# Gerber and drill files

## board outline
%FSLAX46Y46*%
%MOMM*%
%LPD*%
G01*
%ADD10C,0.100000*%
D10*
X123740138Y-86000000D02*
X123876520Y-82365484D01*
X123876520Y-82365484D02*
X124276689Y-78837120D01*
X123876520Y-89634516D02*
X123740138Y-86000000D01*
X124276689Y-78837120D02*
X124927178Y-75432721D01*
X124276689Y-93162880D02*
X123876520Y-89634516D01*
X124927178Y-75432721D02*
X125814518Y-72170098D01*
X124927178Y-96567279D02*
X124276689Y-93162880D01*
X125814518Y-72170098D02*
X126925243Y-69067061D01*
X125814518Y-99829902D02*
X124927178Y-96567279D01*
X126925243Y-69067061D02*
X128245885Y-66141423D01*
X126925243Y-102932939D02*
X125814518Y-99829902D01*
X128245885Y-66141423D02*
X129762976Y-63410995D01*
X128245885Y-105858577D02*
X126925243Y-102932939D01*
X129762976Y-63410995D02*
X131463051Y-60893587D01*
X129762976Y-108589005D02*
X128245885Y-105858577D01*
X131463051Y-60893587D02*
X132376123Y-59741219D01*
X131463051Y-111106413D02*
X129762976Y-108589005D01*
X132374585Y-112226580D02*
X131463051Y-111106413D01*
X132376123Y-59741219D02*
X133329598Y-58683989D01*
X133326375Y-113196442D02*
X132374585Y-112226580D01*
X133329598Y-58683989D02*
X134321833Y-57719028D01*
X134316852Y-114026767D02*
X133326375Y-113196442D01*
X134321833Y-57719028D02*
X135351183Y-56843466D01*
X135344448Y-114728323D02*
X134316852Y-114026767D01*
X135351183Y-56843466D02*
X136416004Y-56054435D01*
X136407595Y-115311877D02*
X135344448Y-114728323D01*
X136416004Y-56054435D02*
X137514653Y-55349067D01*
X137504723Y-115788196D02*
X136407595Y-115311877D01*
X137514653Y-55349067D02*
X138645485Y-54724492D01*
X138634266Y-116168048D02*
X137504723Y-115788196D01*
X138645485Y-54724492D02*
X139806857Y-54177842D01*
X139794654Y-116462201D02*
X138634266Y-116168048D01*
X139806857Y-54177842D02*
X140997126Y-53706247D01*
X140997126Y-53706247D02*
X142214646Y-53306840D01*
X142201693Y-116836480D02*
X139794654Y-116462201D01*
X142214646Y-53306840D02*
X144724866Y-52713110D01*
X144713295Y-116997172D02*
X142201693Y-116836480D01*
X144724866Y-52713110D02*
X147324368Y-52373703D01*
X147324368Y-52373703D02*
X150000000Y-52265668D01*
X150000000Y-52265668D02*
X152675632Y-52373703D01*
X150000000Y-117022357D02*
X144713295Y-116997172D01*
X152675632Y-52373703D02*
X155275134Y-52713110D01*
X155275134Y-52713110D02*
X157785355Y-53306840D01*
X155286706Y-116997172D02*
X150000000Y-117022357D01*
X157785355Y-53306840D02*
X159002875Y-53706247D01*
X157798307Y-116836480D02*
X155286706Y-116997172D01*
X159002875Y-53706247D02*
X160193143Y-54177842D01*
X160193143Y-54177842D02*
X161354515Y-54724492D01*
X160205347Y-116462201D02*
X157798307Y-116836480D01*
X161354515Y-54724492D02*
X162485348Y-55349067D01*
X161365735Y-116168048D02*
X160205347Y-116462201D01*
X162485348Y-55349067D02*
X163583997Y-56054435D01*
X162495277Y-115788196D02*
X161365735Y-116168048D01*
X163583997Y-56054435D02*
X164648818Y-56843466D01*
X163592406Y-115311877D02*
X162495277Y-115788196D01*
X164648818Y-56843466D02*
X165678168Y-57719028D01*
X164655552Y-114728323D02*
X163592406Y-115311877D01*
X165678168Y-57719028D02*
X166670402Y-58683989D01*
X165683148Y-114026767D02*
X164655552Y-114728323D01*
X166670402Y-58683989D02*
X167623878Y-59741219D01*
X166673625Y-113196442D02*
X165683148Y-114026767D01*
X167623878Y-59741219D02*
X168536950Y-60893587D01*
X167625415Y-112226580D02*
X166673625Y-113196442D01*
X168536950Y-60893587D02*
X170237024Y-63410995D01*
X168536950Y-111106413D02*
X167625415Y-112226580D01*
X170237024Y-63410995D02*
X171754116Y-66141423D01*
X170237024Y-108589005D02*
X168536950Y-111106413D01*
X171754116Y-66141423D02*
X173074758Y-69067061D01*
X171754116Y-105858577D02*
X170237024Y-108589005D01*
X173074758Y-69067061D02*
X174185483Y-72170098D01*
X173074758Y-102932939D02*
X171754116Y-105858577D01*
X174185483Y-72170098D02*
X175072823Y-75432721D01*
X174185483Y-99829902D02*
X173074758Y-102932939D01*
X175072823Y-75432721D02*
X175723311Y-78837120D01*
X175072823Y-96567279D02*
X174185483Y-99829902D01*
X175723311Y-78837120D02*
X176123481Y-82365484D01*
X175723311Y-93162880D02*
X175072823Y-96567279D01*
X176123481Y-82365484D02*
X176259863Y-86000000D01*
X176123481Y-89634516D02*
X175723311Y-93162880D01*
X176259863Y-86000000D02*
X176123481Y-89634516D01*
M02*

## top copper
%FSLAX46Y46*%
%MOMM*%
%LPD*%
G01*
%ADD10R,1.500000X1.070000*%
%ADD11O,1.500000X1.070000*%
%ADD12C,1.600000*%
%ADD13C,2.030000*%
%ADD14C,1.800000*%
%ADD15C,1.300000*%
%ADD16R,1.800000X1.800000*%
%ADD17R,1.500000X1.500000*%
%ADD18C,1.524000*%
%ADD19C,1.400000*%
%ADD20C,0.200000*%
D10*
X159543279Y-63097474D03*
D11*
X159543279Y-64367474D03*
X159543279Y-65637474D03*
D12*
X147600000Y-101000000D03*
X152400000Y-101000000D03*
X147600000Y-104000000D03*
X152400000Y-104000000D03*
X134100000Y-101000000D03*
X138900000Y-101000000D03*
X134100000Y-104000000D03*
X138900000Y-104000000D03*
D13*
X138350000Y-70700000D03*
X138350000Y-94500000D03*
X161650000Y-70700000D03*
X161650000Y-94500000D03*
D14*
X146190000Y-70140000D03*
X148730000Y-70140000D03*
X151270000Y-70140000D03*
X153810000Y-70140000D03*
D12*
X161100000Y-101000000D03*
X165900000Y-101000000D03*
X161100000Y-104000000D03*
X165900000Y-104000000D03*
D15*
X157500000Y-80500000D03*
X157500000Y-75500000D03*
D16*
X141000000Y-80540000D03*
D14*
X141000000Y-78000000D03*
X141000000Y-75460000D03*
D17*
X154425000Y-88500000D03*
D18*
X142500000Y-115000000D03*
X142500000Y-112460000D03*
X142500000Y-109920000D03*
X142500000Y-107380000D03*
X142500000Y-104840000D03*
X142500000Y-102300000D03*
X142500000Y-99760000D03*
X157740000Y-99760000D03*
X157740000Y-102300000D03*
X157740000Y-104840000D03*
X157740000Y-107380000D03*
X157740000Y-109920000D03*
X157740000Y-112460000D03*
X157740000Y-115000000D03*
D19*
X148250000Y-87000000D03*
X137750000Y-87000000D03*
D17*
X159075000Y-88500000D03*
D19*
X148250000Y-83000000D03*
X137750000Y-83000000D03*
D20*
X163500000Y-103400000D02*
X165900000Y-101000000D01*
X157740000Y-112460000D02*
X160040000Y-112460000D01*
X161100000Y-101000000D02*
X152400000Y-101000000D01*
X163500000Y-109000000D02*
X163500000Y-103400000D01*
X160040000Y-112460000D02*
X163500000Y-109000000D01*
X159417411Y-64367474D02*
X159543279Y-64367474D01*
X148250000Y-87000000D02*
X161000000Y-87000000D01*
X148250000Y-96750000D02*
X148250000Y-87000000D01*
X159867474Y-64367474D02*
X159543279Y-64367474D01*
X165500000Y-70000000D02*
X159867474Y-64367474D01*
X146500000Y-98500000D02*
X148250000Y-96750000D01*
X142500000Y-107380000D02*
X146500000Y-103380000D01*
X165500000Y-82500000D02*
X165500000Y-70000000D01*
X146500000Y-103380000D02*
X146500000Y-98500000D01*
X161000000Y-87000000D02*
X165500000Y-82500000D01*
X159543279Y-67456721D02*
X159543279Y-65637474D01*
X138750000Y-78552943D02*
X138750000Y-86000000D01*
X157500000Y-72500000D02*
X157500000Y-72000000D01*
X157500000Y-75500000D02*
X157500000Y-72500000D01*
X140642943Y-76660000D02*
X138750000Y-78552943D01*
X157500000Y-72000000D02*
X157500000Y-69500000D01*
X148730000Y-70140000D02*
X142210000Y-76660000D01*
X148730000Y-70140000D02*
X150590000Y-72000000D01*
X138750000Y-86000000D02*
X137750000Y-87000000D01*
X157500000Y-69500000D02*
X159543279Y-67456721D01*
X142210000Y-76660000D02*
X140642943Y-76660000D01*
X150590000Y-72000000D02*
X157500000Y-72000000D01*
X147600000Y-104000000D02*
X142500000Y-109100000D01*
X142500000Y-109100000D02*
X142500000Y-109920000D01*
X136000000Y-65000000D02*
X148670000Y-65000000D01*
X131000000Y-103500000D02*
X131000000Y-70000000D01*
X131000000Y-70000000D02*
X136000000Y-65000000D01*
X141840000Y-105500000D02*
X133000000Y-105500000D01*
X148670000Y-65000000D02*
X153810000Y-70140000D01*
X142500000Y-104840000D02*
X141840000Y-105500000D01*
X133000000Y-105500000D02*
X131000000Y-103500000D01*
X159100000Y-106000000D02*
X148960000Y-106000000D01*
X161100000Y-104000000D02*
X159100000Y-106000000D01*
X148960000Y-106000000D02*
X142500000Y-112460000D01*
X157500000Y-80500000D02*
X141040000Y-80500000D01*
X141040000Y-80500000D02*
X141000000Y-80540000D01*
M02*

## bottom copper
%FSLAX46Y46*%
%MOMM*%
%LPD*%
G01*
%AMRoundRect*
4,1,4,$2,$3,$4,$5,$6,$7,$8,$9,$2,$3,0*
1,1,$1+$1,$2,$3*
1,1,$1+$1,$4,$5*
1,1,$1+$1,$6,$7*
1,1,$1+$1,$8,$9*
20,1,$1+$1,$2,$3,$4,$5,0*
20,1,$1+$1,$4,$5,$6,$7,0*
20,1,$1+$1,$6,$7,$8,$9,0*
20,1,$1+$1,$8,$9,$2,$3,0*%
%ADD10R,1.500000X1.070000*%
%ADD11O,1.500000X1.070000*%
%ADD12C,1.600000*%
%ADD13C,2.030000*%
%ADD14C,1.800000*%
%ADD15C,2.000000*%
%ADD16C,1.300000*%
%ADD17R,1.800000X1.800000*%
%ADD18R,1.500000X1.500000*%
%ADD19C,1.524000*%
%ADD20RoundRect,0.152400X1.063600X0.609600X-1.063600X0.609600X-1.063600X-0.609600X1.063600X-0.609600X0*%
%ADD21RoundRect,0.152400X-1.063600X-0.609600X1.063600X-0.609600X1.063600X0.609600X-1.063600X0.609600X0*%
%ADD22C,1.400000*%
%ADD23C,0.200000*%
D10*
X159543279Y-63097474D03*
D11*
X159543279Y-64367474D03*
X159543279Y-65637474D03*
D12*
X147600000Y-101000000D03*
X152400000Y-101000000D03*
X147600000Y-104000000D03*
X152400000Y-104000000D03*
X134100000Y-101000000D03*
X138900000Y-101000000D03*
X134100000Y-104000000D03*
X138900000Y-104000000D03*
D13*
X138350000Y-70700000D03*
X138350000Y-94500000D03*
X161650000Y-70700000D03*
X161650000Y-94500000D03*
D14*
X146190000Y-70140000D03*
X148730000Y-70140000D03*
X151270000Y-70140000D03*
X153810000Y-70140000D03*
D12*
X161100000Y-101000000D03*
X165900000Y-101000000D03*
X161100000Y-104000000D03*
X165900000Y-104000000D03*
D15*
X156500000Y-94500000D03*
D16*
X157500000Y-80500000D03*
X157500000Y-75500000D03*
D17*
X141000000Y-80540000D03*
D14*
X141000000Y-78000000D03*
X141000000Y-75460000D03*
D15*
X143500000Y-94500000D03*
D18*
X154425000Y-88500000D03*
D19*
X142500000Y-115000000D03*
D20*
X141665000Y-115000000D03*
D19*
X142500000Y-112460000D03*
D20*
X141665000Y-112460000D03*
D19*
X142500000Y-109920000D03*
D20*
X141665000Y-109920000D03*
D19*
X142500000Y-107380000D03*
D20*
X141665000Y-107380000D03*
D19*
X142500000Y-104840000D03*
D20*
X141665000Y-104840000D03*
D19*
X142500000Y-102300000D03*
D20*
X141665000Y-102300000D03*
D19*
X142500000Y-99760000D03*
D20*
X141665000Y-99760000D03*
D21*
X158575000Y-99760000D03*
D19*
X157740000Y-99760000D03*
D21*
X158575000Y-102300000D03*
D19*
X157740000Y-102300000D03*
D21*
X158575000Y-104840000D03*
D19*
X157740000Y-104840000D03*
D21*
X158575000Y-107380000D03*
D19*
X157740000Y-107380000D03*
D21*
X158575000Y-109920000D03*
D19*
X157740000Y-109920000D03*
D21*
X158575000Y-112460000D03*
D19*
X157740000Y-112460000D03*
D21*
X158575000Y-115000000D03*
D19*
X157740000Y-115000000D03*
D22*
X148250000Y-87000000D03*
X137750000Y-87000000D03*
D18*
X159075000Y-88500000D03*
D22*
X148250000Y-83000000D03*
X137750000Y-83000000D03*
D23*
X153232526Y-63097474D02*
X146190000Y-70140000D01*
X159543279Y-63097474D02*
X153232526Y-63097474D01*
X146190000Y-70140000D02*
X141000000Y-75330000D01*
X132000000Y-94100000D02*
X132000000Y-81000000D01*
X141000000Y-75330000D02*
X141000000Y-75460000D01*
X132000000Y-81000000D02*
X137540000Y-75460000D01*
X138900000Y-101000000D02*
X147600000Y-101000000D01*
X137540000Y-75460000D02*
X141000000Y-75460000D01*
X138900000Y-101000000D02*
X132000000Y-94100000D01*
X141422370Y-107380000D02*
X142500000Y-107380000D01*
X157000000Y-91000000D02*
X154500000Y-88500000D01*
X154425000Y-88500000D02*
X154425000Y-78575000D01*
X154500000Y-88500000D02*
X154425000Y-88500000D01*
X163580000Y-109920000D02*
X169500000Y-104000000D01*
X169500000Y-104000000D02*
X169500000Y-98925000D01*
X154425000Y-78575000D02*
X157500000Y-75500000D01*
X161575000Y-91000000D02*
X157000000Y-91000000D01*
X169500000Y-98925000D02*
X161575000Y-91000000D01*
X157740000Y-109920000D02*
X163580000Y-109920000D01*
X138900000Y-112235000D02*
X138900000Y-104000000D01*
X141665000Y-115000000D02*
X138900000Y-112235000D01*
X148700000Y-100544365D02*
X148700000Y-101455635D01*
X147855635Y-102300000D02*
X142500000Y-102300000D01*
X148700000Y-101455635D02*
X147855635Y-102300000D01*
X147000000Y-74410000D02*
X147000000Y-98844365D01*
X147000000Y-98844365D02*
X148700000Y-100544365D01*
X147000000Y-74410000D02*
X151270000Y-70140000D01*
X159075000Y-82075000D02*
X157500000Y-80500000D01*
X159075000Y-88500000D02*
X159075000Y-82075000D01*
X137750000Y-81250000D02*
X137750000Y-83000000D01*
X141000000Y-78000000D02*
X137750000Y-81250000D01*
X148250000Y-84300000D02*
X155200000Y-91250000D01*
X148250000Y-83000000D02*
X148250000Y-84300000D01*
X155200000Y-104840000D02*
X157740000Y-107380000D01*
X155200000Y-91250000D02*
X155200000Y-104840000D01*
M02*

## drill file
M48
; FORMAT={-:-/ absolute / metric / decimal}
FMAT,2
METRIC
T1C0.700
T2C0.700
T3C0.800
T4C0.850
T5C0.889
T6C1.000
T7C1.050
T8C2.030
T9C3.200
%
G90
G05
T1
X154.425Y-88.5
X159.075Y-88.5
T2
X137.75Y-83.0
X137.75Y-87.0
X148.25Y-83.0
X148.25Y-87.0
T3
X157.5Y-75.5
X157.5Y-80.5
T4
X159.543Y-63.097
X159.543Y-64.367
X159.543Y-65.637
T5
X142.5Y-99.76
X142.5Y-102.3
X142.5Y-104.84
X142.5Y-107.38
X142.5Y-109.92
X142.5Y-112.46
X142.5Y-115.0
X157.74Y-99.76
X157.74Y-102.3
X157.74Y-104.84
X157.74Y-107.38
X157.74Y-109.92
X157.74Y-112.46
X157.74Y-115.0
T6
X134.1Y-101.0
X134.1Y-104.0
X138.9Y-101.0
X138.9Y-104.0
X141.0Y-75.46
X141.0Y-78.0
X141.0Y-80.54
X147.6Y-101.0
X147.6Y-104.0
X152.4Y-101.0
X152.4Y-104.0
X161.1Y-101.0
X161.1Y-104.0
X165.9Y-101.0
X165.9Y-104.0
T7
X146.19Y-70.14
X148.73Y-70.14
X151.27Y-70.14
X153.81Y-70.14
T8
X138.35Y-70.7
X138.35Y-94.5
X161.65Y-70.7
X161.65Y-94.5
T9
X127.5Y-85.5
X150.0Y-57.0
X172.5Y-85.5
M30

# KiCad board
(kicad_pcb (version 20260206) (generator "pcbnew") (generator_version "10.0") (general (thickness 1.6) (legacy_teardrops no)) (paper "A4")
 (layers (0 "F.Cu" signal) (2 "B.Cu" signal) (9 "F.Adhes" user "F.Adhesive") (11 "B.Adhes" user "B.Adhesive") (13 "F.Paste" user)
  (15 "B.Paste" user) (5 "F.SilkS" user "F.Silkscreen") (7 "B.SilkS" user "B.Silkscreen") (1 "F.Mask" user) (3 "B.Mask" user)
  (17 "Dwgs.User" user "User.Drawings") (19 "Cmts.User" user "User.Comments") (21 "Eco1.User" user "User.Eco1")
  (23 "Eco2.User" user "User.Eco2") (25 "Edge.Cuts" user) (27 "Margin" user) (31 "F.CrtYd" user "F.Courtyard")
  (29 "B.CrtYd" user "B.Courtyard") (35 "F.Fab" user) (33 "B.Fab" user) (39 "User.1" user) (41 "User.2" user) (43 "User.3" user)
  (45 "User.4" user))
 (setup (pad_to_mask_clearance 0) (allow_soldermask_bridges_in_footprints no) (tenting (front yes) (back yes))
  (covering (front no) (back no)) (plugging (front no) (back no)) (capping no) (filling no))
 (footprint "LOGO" (layer "F.Cu") (at 140.5 63)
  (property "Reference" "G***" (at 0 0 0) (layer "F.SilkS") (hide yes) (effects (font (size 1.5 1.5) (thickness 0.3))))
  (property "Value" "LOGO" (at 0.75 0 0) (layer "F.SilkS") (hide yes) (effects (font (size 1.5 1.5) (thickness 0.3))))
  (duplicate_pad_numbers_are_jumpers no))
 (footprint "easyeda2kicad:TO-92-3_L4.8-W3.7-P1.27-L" (layer "F.Cu") (at 159.543279 64.367474 -90)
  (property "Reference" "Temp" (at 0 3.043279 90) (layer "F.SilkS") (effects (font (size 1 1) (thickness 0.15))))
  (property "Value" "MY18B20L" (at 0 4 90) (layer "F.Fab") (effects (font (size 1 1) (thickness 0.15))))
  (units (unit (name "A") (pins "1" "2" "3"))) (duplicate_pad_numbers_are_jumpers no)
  (pad "1" thru_hole rect (at -1.27 0 270) (size 1.07 1.5) (drill 0.849986) (layers "*.Cu" "*.Mask") (remove_unused_layers no) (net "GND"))
  (pad "2" thru_hole oval (at 0 0 270) (size 1.07 1.5) (drill 0.849986) (layers "*.Cu" "*.Mask") (remove_unused_layers no)
   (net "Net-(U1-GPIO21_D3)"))
  (pad "3" thru_hole oval (at 1.27 0 270) (size 1.07 1.5) (drill 0.849986) (layers "*.Cu" "*.Mask") (remove_unused_layers no) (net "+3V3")))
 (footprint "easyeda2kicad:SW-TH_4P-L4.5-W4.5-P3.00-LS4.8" (layer "F.Cu") (at 150 102.5)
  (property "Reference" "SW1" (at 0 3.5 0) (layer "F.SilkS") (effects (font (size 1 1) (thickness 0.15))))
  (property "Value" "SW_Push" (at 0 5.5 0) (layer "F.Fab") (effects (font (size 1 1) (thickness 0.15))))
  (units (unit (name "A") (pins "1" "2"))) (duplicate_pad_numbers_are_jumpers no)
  (pad "1" thru_hole circle (at -2.4 -1.5) (size 1.6 1.6) (drill 0.999998) (layers "*.Cu" "*.Mask") (remove_unused_layers no) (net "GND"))
  (pad "1" thru_hole circle (at 2.4 -1.5) (size 1.6 1.6) (drill 0.999998) (layers "*.Cu" "*.Mask") (remove_unused_layers no) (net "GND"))
  (pad "2" thru_hole circle (at -2.4 1.5) (size 1.6 1.6) (drill 0.999998) (layers "*.Cu" "*.Mask") (remove_unused_layers no)
   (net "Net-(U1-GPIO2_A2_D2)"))
  (pad "2" thru_hole circle (at 2.4 1.5) (size 1.6 1.6) (drill 0.999998) (layers "*.Cu" "*.Mask") (remove_unused_layers no)
   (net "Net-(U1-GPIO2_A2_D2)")))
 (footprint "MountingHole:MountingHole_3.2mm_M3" (layer "F.Cu") (at 172.5 85.5)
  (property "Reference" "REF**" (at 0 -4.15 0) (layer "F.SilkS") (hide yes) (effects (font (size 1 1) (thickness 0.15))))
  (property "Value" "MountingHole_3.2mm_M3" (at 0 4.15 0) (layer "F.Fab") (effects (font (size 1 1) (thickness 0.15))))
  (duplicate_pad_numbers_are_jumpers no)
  (pad "" np_thru_hole circle (at 0 0) (size 3.2 3.2) (drill 3.2) (layers "*.Cu" "*.Mask")))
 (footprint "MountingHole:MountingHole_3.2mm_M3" (layer "F.Cu") (at 127.5 85.5)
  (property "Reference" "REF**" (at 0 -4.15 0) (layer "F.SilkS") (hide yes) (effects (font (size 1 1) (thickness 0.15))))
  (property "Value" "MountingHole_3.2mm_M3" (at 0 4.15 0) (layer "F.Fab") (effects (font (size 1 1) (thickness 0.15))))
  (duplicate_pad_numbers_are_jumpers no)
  (pad "" np_thru_hole circle (at 0 0) (size 3.2 3.2) (drill 3.2) (layers "*.Cu" "*.Mask")))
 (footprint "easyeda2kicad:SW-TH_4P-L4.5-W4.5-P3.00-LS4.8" (layer "F.Cu") (at 136.5 102.5)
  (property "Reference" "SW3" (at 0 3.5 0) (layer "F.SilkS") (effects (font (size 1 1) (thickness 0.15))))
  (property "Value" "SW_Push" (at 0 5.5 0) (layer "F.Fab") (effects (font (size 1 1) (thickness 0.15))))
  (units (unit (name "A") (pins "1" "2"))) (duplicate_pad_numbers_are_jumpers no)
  (pad "1" thru_hole circle (at -2.4 -1.5) (size 1.6 1.6) (drill 0.999998) (layers "*.Cu" "*.Mask") (remove_unused_layers no) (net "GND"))
  (pad "1" thru_hole circle (at 2.4 -1.5) (size 1.6 1.6) (drill 0.999998) (layers "*.Cu" "*.Mask") (remove_unused_layers no) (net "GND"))
  (pad "2" thru_hole circle (at -2.4 1.5) (size 1.6 1.6) (drill 0.999998) (layers "*.Cu" "*.Mask") (remove_unused_layers no)
   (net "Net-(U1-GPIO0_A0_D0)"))
  (pad "2" thru_hole circle (at 2.4 1.5) (size 1.6 1.6) (drill 0.999998) (layers "*.Cu" "*.Mask") (remove_unused_layers no)
   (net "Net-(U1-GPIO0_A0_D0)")))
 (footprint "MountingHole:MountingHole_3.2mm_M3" (layer "F.Cu") (at 150 57)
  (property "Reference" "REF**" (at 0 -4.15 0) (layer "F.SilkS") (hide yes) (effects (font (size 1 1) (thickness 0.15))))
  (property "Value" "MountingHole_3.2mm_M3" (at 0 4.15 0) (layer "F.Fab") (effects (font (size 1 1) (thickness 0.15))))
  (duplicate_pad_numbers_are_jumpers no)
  (pad "" np_thru_hole circle (at 0 0) (size 3.2 3.2) (drill 3.2) (layers "*.Cu" "*.Mask")))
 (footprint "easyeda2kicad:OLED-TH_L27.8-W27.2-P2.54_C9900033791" (layer "F.Cu") (at 150 70.14)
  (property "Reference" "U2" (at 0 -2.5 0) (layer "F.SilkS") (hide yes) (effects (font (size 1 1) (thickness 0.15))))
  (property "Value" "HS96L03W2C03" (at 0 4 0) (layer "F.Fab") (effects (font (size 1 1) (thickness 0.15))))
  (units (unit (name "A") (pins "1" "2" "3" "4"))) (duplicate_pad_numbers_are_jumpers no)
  (pad "" thru_hole circle (at -11.65 0.56) (size 2.03 2.03) (drill 2.03) (layers "*.Cu" "*.Mask") (remove_unused_layers no))
  (pad "" thru_hole circle (at -11.65 24.36) (size 2.03 2.03) (drill 2.03) (layers "*.Cu" "*.Mask") (remove_unused_layers no))
  (pad "" thru_hole circle (at 11.65 0.56) (size 2.03 2.03) (drill 2.03) (layers "*.Cu" "*.Mask") (remove_unused_layers no))
  (pad "" thru_hole circle (at 11.65 24.36) (size 2.03 2.03) (drill 2.03) (layers "*.Cu" "*.Mask") (remove_unused_layers no))
  (pad "1" thru_hole circle (at -3.81 0) (size 1.8 1.8) (drill 1.049985) (layers "*.Cu" "*.Mask") (remove_unused_layers no) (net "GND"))
  (pad "2" thru_hole circle (at -1.27 0) (size 1.8 1.8) (drill 1.049985) (layers "*.Cu" "*.Mask") (remove_unused_layers no) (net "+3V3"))
  (pad "3" thru_hole circle (at 1.27 0) (size 1.8 1.8) (drill 1.049985) (layers "*.Cu" "*.Mask") (remove_unused_layers no)
   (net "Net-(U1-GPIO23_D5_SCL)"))
  (pad "4" thru_hole circle (at 3.81 0) (size 1.8 1.8) (drill 1.049985) (layers "*.Cu" "*.Mask") (remove_unused_layers no)
   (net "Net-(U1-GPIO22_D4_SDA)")))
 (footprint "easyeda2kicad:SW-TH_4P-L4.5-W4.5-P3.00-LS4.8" (layer "F.Cu") (at 163.5 102.5)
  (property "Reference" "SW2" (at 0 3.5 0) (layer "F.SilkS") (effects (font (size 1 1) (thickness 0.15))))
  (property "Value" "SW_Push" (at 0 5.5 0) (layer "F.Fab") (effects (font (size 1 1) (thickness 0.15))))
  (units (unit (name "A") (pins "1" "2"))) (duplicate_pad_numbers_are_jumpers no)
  (pad "1" thru_hole circle (at -2.4 -1.5) (size 1.6 1.6) (drill 0.999998) (layers "*.Cu" "*.Mask") (remove_unused_layers no) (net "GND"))
  (pad "1" thru_hole circle (at 2.4 -1.5) (size 1.6 1.6) (drill 0.999998) (layers "*.Cu" "*.Mask") (remove_unused_layers no) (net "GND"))
  (pad "2" thru_hole circle (at -2.4 1.5) (size 1.6 1.6) (drill 0.999998) (layers "*.Cu" "*.Mask") (remove_unused_layers no)
   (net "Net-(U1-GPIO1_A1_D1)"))
  (pad "2" thru_hole circle (at 2.4 1.5) (size 1.6 1.6) (drill 0.999998) (layers "*.Cu" "*.Mask") (remove_unused_layers no)
   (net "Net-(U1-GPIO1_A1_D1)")))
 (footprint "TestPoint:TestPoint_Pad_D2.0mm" (layer "B.Cu") (at 156.5 94.5 180)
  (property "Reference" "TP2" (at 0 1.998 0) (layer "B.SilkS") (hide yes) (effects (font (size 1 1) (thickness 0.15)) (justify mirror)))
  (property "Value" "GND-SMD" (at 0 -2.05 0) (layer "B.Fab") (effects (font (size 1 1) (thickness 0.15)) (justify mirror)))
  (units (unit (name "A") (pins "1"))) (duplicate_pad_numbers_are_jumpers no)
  (pad "1" smd circle (at 0 0 180) (size 2 2) (layers "B.Cu" "B.Mask") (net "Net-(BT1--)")))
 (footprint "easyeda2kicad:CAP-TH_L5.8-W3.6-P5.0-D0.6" (layer "B.Cu") (at 157.5 78 90)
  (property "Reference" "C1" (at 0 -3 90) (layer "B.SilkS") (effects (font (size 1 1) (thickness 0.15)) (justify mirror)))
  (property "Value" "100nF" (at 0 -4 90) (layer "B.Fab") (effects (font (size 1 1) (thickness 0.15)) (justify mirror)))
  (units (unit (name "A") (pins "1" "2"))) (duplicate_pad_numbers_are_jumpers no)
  (pad "1" thru_hole circle (at -2.5 0 90) (size 1.3 1.3) (drill 0.799998) (layers "*.Cu" "*.Mask") (remove_unused_layers no)
   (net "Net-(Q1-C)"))
  (pad "2" thru_hole circle (at 2.5 0 90) (size 1.3 1.3) (drill 0.799998) (layers "*.Cu" "*.Mask") (remove_unused_layers no) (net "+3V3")))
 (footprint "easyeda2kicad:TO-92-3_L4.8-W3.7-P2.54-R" (layer "B.Cu") (at 141 78 -90)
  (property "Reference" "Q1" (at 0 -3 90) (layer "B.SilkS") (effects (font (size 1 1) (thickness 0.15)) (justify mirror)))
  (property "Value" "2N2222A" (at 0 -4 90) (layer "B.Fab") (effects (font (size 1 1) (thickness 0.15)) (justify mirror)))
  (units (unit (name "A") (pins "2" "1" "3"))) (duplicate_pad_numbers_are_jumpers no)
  (pad "1" thru_hole rect (at 2.54 0) (size 1.8 1.8) (drill 0.999998) (layers "*.Cu" "*.Mask") (remove_unused_layers no) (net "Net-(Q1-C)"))
  (pad "2" thru_hole circle (at 0 0) (size 1.8 1.8) (drill 0.999998) (layers "*.Cu" "*.Mask") (remove_unused_layers no) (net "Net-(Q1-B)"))
  (pad "3" thru_hole circle (at -2.54 0) (size 1.8 1.8) (drill 0.999998) (layers "*.Cu" "*.Mask") (remove_unused_layers no) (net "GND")))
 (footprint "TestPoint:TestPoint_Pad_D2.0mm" (layer "B.Cu") (at 143.5 94.5 180)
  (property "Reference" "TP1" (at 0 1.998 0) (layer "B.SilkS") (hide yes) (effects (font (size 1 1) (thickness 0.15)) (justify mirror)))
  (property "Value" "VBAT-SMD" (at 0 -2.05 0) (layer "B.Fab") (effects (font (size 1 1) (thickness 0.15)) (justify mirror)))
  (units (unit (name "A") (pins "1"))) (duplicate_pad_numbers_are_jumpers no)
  (pad "1" smd circle (at 0 0 180) (size 2 2) (layers "B.Cu" "B.Mask") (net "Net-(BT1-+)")))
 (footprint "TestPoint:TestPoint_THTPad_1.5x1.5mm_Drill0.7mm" (layer "B.Cu") (at 154.425 88.5 90)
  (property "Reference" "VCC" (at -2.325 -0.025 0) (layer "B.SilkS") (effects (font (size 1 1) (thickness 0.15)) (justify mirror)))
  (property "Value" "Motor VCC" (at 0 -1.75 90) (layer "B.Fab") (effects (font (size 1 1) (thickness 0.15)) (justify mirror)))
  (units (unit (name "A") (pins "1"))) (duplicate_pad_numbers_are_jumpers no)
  (pad "1" thru_hole rect (at 0 0 90) (size 1.5 1.5) (drill 0.7) (layers "*.Cu" "*.Mask") (remove_unused_layers no) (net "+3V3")))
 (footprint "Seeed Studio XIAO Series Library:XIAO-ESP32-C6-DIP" (layer "B.Cu") (at 150.12 107.38 -90)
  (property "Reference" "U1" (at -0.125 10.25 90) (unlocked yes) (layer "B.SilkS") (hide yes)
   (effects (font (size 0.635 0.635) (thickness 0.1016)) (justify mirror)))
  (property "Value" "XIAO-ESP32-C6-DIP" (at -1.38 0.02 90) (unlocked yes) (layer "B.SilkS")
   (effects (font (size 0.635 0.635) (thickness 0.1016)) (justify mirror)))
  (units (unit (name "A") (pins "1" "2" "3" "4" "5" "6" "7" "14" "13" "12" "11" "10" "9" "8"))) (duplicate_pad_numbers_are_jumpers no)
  (pad "1" thru_hole circle (at 7.62 7.62 180) (size 1.524 1.524) (drill 0.889) (layers "*.Cu" "*.Mask") (remove_unused_layers no)
   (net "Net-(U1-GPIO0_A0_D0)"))
  (pad "1" smd roundrect (at 7.62 8.455 180) (size 2.432 1.524) (layers "B.Cu" "B.Mask") (roundrect_rratio 0.1) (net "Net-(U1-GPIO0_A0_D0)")
   (thermal_bridge_angle 45))
  (pad "2" thru_hole circle (at 5.08 7.62 180) (size 1.524 1.524) (drill 0.889) (layers "*.Cu" "*.Mask") (remove_unused_layers no)
   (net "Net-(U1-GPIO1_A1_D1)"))
  (pad "2" smd roundrect (at 5.08 8.455 180) (size 2.432 1.524) (layers "B.Cu" "B.Mask") (roundrect_rratio 0.1) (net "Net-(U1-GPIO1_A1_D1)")
   (thermal_bridge_angle 45))
  (pad "3" thru_hole circle (at 2.54 7.62 180) (size 1.524 1.524) (drill 0.889) (layers "*.Cu" "*.Mask") (remove_unused_layers no)
   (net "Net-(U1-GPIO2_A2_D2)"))
  (pad "3" smd roundrect (at 2.54 8.455 180) (size 2.432 1.524) (layers "B.Cu" "B.Mask") (roundrect_rratio 0.1) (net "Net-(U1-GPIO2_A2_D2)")
   (thermal_bridge_angle 45))
  (pad "4" thru_hole circle (at 0 7.62 180) (size 1.524 1.524) (drill 0.889) (layers "*.Cu" "*.Mask") (remove_unused_layers no)
   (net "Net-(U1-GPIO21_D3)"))
  (pad "4" smd roundrect (at 0 8.455 180) (size 2.432 1.524) (layers "B.Cu" "B.Mask") (roundrect_rratio 0.1) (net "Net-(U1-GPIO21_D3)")
   (thermal_bridge_angle 45))
  (pad "5" thru_hole circle (at -2.54 7.62 180) (size 1.524 1.524) (drill 0.889) (layers "*.Cu" "*.Mask") (remove_unused_layers no)
   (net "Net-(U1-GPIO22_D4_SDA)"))
  (pad "5" smd roundrect (at -2.54 8.455 180) (size 2.432 1.524) (layers "B.Cu" "B.Mask") (roundrect_rratio 0.1)
   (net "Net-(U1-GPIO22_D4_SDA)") (thermal_bridge_angle 45))
  (pad "6" thru_hole circle (at -5.08 7.62 180) (size 1.524 1.524) (drill 0.889) (layers "*.Cu" "*.Mask") (remove_unused_layers no)
   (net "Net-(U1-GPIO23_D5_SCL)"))
  (pad "6" smd roundrect (at -5.08 8.455 180) (size 2.432 1.524) (layers "B.Cu" "B.Mask") (roundrect_rratio 0.1)
   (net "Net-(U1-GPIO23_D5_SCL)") (thermal_bridge_angle 45))
  (pad "7" thru_hole circle (at -7.62 7.62 180) (size 1.524 1.524) (drill 0.889) (layers "*.Cu" "*.Mask") (remove_unused_layers no)
   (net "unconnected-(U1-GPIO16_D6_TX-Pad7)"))
  (pad "7" smd roundrect (at -7.62 8.455 180) (size 2.432 1.524) (layers "B.Cu" "B.Mask") (roundrect_rratio 0.1)
   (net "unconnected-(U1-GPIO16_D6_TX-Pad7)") (thermal_bridge_angle 45))
  (pad "8" smd roundrect (at -7.62 -8.455) (size 2.432 1.524) (layers "B.Cu" "B.Mask") (roundrect_rratio 0.1)
   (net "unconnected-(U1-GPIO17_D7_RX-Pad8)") (thermal_bridge_angle 45))
  (pad "8" thru_hole circle (at -7.62 -7.62) (size 1.524 1.524) (drill 0.889) (layers "*.Cu" "*.Mask") (remove_unused_layers no)
   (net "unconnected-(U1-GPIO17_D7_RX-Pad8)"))
  (pad "9" smd roundrect (at -5.08 -8.455) (size 2.432 1.524) (layers "B.Cu" "B.Mask") (roundrect_rratio 0.1)
   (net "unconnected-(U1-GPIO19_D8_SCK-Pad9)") (thermal_bridge_angle 45))
  (pad "9" thru_hole circle (at -5.08 -7.62) (size 1.524 1.524) (drill 0.889) (layers "*.Cu" "*.Mask") (remove_unused_layers no)
   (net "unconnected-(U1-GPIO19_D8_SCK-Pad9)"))
  (pad "10" smd roundrect (at -2.54 -8.455) (size 2.432 1.524) (layers "B.Cu" "B.Mask") (roundrect_rratio 0.1)
   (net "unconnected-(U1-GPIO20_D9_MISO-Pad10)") (thermal_bridge_angle 45))
  (pad "10" thru_hole circle (at -2.54 -7.62) (size 1.524 1.524) (drill 0.889) (layers "*.Cu" "*.Mask") (remove_unused_layers no)
   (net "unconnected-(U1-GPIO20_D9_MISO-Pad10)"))
  (pad "11" smd roundrect (at 0 -8.455) (size 2.432 1.524) (layers "B.Cu" "B.Mask") (roundrect_rratio 0.1) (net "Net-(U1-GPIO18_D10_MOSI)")
   (thermal_bridge_angle 45))
  (pad "11" thru_hole circle (at 0 -7.62) (size 1.524 1.524) (drill 0.889) (layers "*.Cu" "*.Mask") (remove_unused_layers no)
   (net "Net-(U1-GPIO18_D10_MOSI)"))
  (pad "12" smd roundrect (at 2.54 -8.455) (size 2.432 1.524) (layers "B.Cu" "B.Mask") (roundrect_rratio 0.1) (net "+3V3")
   (thermal_bridge_angle 45))
  (pad "12" thru_hole circle (at 2.54 -7.62) (size 1.524 1.524) (drill 0.889) (layers "*.Cu" "*.Mask") (remove_unused_layers no)
   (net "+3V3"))
  (pad "13" smd roundrect (at 5.08 -8.455) (size 2.432 1.524) (layers "B.Cu" "B.Mask") (roundrect_rratio 0.1) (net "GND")
   (thermal_bridge_angle 45))
  (pad "13" thru_hole circle (at 5.08 -7.62) (size 1.524 1.524) (drill 0.889) (layers "*.Cu" "*.Mask") (remove_unused_layers no) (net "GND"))
  (pad "14" smd roundrect (at 7.62 -8.455) (size 2.432 1.524) (layers "B.Cu" "B.Mask") (roundrect_rratio 0.1) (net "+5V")
   (thermal_bridge_angle 45))
  (pad "14" thru_hole circle (at 7.62 -7.62) (size 1.524 1.524) (drill 0.889) (layers "*.Cu" "*.Mask") (remove_unused_layers no) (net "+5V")))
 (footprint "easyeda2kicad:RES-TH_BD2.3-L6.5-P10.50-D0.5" (layer "B.Cu") (at 143 87 180)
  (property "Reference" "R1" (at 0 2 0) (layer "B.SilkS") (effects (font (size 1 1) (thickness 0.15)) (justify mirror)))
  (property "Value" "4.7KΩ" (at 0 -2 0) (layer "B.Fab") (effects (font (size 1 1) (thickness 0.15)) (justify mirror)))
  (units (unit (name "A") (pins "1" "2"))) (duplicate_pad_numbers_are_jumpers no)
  (pad "1" thru_hole circle (at -5.25 0 180) (size 1.4 1.4) (drill 0.700024) (layers "*.Cu" "*.Mask") (remove_unused_layers no)
   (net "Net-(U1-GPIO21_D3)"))
  (pad "2" thru_hole circle (at 5.25 0 180) (size 1.4 1.4) (drill 0.700024) (layers "*.Cu" "*.Mask") (remove_unused_layers no) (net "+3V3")))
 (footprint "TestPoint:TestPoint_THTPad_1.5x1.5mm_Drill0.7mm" (layer "B.Cu") (at 159.075 88.5 90)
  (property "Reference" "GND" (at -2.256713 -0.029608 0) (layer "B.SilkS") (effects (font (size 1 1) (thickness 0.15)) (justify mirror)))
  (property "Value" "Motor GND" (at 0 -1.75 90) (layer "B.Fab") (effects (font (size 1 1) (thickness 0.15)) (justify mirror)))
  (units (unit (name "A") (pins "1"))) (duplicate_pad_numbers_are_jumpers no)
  (pad "1" thru_hole rect (at 0 0 90) (size 1.5 1.5) (drill 0.7) (layers "*.Cu" "*.Mask") (remove_unused_layers no) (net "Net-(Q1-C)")))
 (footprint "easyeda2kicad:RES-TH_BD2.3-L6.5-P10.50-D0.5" (layer "B.Cu") (at 143 83 180)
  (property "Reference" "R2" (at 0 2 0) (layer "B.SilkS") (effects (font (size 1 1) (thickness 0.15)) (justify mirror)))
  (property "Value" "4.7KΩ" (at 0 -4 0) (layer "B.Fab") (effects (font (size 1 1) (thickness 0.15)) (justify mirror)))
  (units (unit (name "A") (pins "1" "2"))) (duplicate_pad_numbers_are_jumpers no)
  (pad "1" thru_hole circle (at -5.25 0 180) (size 1.4 1.4) (drill 0.700024) (layers "*.Cu" "*.Mask") (remove_unused_layers no)
   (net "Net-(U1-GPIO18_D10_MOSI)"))
  (pad "2" thru_hole circle (at 5.25 0 180) (size 1.4 1.4) (drill 0.700024) (layers "*.Cu" "*.Mask") (remove_unused_layers no)
   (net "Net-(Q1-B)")))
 (gr_line (start 123.740138 86) (end 123.87652 82.365484) (stroke (width 0.1) (type default)) (layer "Edge.Cuts"))
 (gr_line (start 123.87652 82.365484) (end 124.276689 78.83712) (stroke (width 0.1) (type default)) (layer "Edge.Cuts"))
 (gr_line (start 123.87652 89.634516) (end 123.740138 86) (stroke (width 0.1) (type default)) (layer "Edge.Cuts"))
 (gr_line (start 124.276689 78.83712) (end 124.927178 75.432721) (stroke (width 0.1) (type default)) (layer "Edge.Cuts"))
 (gr_line (start 124.276689 93.16288) (end 123.87652 89.634516) (stroke (width 0.1) (type default)) (layer "Edge.Cuts"))
 (gr_line (start 124.927178 75.432721) (end 125.814518 72.170098) (stroke (width 0.1) (type default)) (layer "Edge.Cuts"))
 (gr_line (start 124.927178 96.567279) (end 124.276689 93.16288) (stroke (width 0.1) (type default)) (layer "Edge.Cuts"))
 (gr_line (start 125.814518 72.170098) (end 126.925243 69.067061) (stroke (width 0.1) (type default)) (layer "Edge.Cuts"))
 (gr_line (start 125.814518 99.829902) (end 124.927178 96.567279) (stroke (width 0.1) (type default)) (layer "Edge.Cuts"))
 (gr_line (start 126.925243 69.067061) (end 128.245885 66.141423) (stroke (width 0.1) (type default)) (layer "Edge.Cuts"))
 (gr_line (start 126.925243 102.932939) (end 125.814518 99.829902) (stroke (width 0.1) (type default)) (layer "Edge.Cuts"))
 (gr_line (start 128.245885 66.141423) (end 129.762976 63.410995) (stroke (width 0.1) (type default)) (layer "Edge.Cuts"))
 (gr_line (start 128.245885 105.858577) (end 126.925243 102.932939) (stroke (width 0.1) (type default)) (layer "Edge.Cuts"))
 (gr_line (start 129.762976 63.410995) (end 131.463051 60.893587) (stroke (width 0.1) (type default)) (layer "Edge.Cuts"))
 (gr_line (start 129.762976 108.589005) (end 128.245885 105.858577) (stroke (width 0.1) (type default)) (layer "Edge.Cuts"))
 (gr_line (start 131.463051 60.893587) (end 132.376123 59.741219) (stroke (width 0.1) (type default)) (layer "Edge.Cuts"))
 (gr_line (start 131.463051 111.106413) (end 129.762976 108.589005) (stroke (width 0.1) (type default)) (layer "Edge.Cuts"))
 (gr_line (start 132.374585 112.22658) (end 131.463051 111.106413) (stroke (width 0.1) (type default)) (layer "Edge.Cuts"))
 (gr_line (start 132.376123 59.741219) (end 133.329598 58.683989) (stroke (width 0.1) (type default)) (layer "Edge.Cuts"))
 (gr_line (start 133.326375 113.196442) (end 132.374585 112.22658) (stroke (width 0.1) (type default)) (layer "Edge.Cuts"))
 (gr_line (start 133.329598 58.683989) (end 134.321833 57.719028) (stroke (width 0.1) (type default)) (layer "Edge.Cuts"))
 (gr_line (start 134.316852 114.026767) (end 133.326375 113.196442) (stroke (width 0.1) (type default)) (layer "Edge.Cuts"))
 (gr_line (start 134.321833 57.719028) (end 135.351183 56.843466) (stroke (width 0.1) (type default)) (layer "Edge.Cuts"))
 (gr_line (start 135.344448 114.728323) (end 134.316852 114.026767) (stroke (width 0.1) (type default)) (layer "Edge.Cuts"))
 (gr_line (start 135.351183 56.843466) (end 136.416004 56.054435) (stroke (width 0.1) (type default)) (layer "Edge.Cuts"))
 (gr_line (start 136.407595 115.311877) (end 135.344448 114.728323) (stroke (width 0.1) (type default)) (layer "Edge.Cuts"))
 (gr_line (start 136.416004 56.054435) (end 137.514653 55.349067) (stroke (width 0.1) (type default)) (layer "Edge.Cuts"))
 (gr_line (start 137.504723 115.788196) (end 136.407595 115.311877) (stroke (width 0.1) (type default)) (layer "Edge.Cuts"))
 (gr_line (start 137.514653 55.349067) (end 138.645485 54.724492) (stroke (width 0.1) (type default)) (layer "Edge.Cuts"))
 (gr_line (start 138.634266 116.168048) (end 137.504723 115.788196) (stroke (width 0.1) (type default)) (layer "Edge.Cuts"))
 (gr_line (start 138.645485 54.724492) (end 139.806857 54.177842) (stroke (width 0.1) (type default)) (layer "Edge.Cuts"))
 (gr_line (start 139.794654 116.462201) (end 138.634266 116.168048) (stroke (width 0.1) (type default)) (layer "Edge.Cuts"))
 (gr_line (start 139.806857 54.177842) (end 140.997126 53.706247) (stroke (width 0.1) (type default)) (layer "Edge.Cuts"))
 (gr_line (start 140.997126 53.706247) (end 142.214646 53.30684) (stroke (width 0.1) (type default)) (layer "Edge.Cuts"))
 (gr_line (start 142.201693 116.83648) (end 139.794654 116.462201) (stroke (width 0.1) (type default)) (layer "Edge.Cuts"))
 (gr_line (start 142.214646 53.30684) (end 144.724866 52.71311) (stroke (width 0.1) (type default)) (layer "Edge.Cuts"))
 (gr_line (start 144.713295 116.997172) (end 142.201693 116.83648) (stroke (width 0.1) (type default)) (layer "Edge.Cuts"))
 (gr_line (start 144.724866 52.71311) (end 147.324368 52.373703) (stroke (width 0.1) (type default)) (layer "Edge.Cuts"))
 (gr_line (start 147.324368 52.373703) (end 150 52.265668) (stroke (width 0.1) (type default)) (layer "Edge.Cuts"))
 (gr_line (start 150 52.265668) (end 152.675632 52.373703) (stroke (width 0.1) (type default)) (layer "Edge.Cuts"))
 (gr_line (start 150 117.022357) (end 144.713295 116.997172) (stroke (width 0.1) (type default)) (layer "Edge.Cuts"))
 (gr_line (start 152.675632 52.373703) (end 155.275134 52.71311) (stroke (width 0.1) (type default)) (layer "Edge.Cuts"))
 (gr_line (start 155.275134 52.71311) (end 157.785355 53.30684) (stroke (width 0.1) (type default)) (layer "Edge.Cuts"))
 (gr_line (start 155.286706 116.997172) (end 150 117.022357) (stroke (width 0.1) (type default)) (layer "Edge.Cuts"))
 (gr_line (start 157.785355 53.30684) (end 159.002875 53.706247) (stroke (width 0.1) (type default)) (layer "Edge.Cuts"))
 (gr_line (start 157.798307 116.83648) (end 155.286706 116.997172) (stroke (width 0.1) (type default)) (layer "Edge.Cuts"))
 (gr_line (start 159.002875 53.706247) (end 160.193143 54.177842) (stroke (width 0.1) (type default)) (layer "Edge.Cuts"))
 (gr_line (start 160.193143 54.177842) (end 161.354515 54.724492) (stroke (width 0.1) (type default)) (layer "Edge.Cuts"))
 (gr_line (start 160.205347 116.462201) (end 157.798307 116.83648) (stroke (width 0.1) (type default)) (layer "Edge.Cuts"))
 (gr_line (start 161.354515 54.724492) (end 162.485348 55.349067) (stroke (width 0.1) (type default)) (layer "Edge.Cuts"))
 (gr_line (start 161.365735 116.168048) (end 160.205347 116.462201) (stroke (width 0.1) (type default)) (layer "Edge.Cuts"))
 (gr_line (start 162.485348 55.349067) (end 163.583997 56.054435) (stroke (width 0.1) (type default)) (layer "Edge.Cuts"))
 (gr_line (start 162.495277 115.788196) (end 161.365735 116.168048) (stroke (width 0.1) (type default)) (layer "Edge.Cuts"))
 (gr_line (start 163.583997 56.054435) (end 164.648818 56.843466) (stroke (width 0.1) (type default)) (layer "Edge.Cuts"))
 (gr_line (start 163.592406 115.311877) (end 162.495277 115.788196) (stroke (width 0.1) (type default)) (layer "Edge.Cuts"))
 (gr_line (start 164.648818 56.843466) (end 165.678168 57.719028) (stroke (width 0.1) (type default)) (layer "Edge.Cuts"))
 (gr_line (start 164.655552 114.728323) (end 163.592406 115.311877) (stroke (width 0.1) (type default)) (layer "Edge.Cuts"))
 (gr_line (start 165.678168 57.719028) (end 166.670402 58.683989) (stroke (width 0.1) (type default)) (layer "Edge.Cuts"))
 (gr_line (start 165.683148 114.026767) (end 164.655552 114.728323) (stroke (width 0.1) (type default)) (layer "Edge.Cuts"))
 (gr_line (start 166.670402 58.683989) (end 167.623878 59.741219) (stroke (width 0.1) (type default)) (layer "Edge.Cuts"))
 (gr_line (start 166.673625 113.196442) (end 165.683148 114.026767) (stroke (width 0.1) (type default)) (layer "Edge.Cuts"))
 (gr_line (start 167.623878 59.741219) (end 168.53695 60.893587) (stroke (width 0.1) (type default)) (layer "Edge.Cuts"))
 (gr_line (start 167.625415 112.22658) (end 166.673625 113.196442) (stroke (width 0.1) (type default)) (layer "Edge.Cuts"))
 (gr_line (start 168.53695 60.893587) (end 170.237024 63.410995) (stroke (width 0.1) (type default)) (layer "Edge.Cuts"))
 (gr_line (start 168.53695 111.106413) (end 167.625415 112.22658) (stroke (width 0.1) (type default)) (layer "Edge.Cuts"))
 (gr_line (start 170.237024 63.410995) (end 171.754116 66.141423) (stroke (width 0.1) (type default)) (layer "Edge.Cuts"))
 (gr_line (start 170.237024 108.589005) (end 168.53695 111.106413) (stroke (width 0.1) (type default)) (layer "Edge.Cuts"))
 (gr_line (start 171.754116 66.141423) (end 173.074758 69.067061) (stroke (width 0.1) (type default)) (layer "Edge.Cuts"))
 (gr_line (start 171.754116 105.858577) (end 170.237024 108.589005) (stroke (width 0.1) (type default)) (layer "Edge.Cuts"))
 (gr_line (start 173.074758 69.067061) (end 174.185483 72.170098) (stroke (width 0.1) (type default)) (layer "Edge.Cuts"))
 (gr_line (start 173.074758 102.932939) (end 171.754116 105.858577) (stroke (width 0.1) (type default)) (layer "Edge.Cuts"))
 (gr_line (start 174.185483 72.170098) (end 175.072823 75.432721) (stroke (width 0.1) (type default)) (layer "Edge.Cuts"))
 (gr_line (start 174.185483 99.829902) (end 173.074758 102.932939) (stroke (width 0.1) (type default)) (layer "Edge.Cuts"))
 (gr_line (start 175.072823 75.432721) (end 175.723311 78.83712) (stroke (width 0.1) (type default)) (layer "Edge.Cuts"))
 (gr_line (start 175.072823 96.567279) (end 174.185483 99.829902) (stroke (width 0.1) (type default)) (layer "Edge.Cuts"))
 (gr_line (start 175.723311 78.83712) (end 176.123481 82.365484) (stroke (width 0.1) (type default)) (layer "Edge.Cuts"))
 (gr_line (start 175.723311 93.16288) (end 175.072823 96.567279) (stroke (width 0.1) (type default)) (layer "Edge.Cuts"))
 (gr_line (start 176.123481 82.365484) (end 176.259863 86) (stroke (width 0.1) (type default)) (layer "Edge.Cuts"))
 (gr_line (start 176.123481 89.634516) (end 175.723311 93.16288) (stroke (width 0.1) (type default)) (layer "Edge.Cuts"))
 (gr_line (start 176.259863 86) (end 176.123481 89.634516) (stroke (width 0.1) (type default)) (layer "Edge.Cuts"))
 (segment (start 163.5 103.4) (end 165.9 101) (width 0.2) (layer "F.Cu") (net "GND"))
 (segment (start 157.74 112.46) (end 160.04 112.46) (width 0.2) (layer "F.Cu") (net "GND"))
 (segment (start 161.1 101) (end 152.4 101) (width 0.2) (layer "F.Cu") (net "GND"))
 (segment (start 163.5 109) (end 163.5 103.4) (width 0.2) (layer "F.Cu") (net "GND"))
 (segment (start 160.04 112.46) (end 163.5 109) (width 0.2) (layer "F.Cu") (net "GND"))
 (segment (start 153.232526 63.097474) (end 146.19 70.14) (width 0.2) (layer "B.Cu") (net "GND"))
 (segment (start 159.543279 63.097474) (end 153.232526 63.097474) (width 0.2) (layer "B.Cu") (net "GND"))
 (segment (start 146.19 70.14) (end 141 75.33) (width 0.2) (layer "B.Cu") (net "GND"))
 (segment (start 132 94.1) (end 132 81) (width 0.2) (layer "B.Cu") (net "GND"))
 (segment (start 141 75.33) (end 141 75.46) (width 0.2) (layer "B.Cu") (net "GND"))
 (segment (start 132 81) (end 137.54 75.46) (width 0.2) (layer "B.Cu") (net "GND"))
 (segment (start 138.9 101) (end 147.6 101) (width 0.2) (layer "B.Cu") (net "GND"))
 (segment (start 137.54 75.46) (end 141 75.46) (width 0.2) (layer "B.Cu") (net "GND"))
 (segment (start 138.9 101) (end 132 94.1) (width 0.2) (layer "B.Cu") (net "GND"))
 (segment (start 159.417411 64.367474) (end 159.543279 64.367474) (width 0.2) (layer "F.Cu") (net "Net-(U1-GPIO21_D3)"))
 (segment (start 148.25 87) (end 161 87) (width 0.2) (layer "F.Cu") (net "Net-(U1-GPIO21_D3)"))
 (segment (start 148.25 96.75) (end 148.25 87) (width 0.2) (layer "F.Cu") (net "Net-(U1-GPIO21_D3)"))
 (segment (start 159.867474 64.367474) (end 159.543279 64.367474) (width 0.2) (layer "F.Cu") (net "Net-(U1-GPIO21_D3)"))
 (segment (start 165.5 70) (end 159.867474 64.367474) (width 0.2) (layer "F.Cu") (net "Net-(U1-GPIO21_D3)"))
 (segment (start 146.5 98.5) (end 148.25 96.75) (width 0.2) (layer "F.Cu") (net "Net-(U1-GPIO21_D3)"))
 (segment (start 142.5 107.38) (end 146.5 103.38) (width 0.2) (layer "F.Cu") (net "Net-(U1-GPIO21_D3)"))
 (segment (start 165.5 82.5) (end 165.5 70) (width 0.2) (layer "F.Cu") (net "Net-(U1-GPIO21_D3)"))
 (segment (start 146.5 103.38) (end 146.5 98.5) (width 0.2) (layer "F.Cu") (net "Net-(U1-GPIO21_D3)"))
 (segment (start 161 87) (end 165.5 82.5) (width 0.2) (layer "F.Cu") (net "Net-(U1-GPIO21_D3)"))
 (segment (start 141.42237 107.38) (end 142.5 107.38) (width 0.2) (layer "B.Cu") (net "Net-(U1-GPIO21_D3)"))
 (segment (start 159.543279 67.456721) (end 159.543279 65.637474) (width 0.2) (layer "F.Cu") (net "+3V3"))
 (segment (start 138.75 78.552943) (end 138.75 86) (width 0.2) (layer "F.Cu") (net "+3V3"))
 (segment (start 157.5 72.5) (end 157.5 72) (width 0.2) (layer "F.Cu") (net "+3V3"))
 (segment (start 157.5 75.5) (end 157.5 72.5) (width 0.2) (layer "F.Cu") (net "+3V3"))
 (segment (start 140.642943 76.66) (end 138.75 78.552943) (width 0.2) (layer "F.Cu") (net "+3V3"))
 (segment (start 157.5 72) (end 157.5 69.5) (width 0.2) (layer "F.Cu") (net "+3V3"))
 (segment (start 148.73 70.14) (end 142.21 76.66) (width 0.2) (layer "F.Cu") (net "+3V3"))
 (segment (start 148.73 70.14) (end 150.59 72) (width 0.2) (layer "F.Cu") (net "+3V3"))
 (segment (start 138.75 86) (end 137.75 87) (width 0.2) (layer "F.Cu") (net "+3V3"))
 (segment (start 157.5 69.5) (end 159.543279 67.456721) (width 0.2) (layer "F.Cu") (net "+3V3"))
 (segment (start 142.21 76.66) (end 140.642943 76.66) (width 0.2) (layer "F.Cu") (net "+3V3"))
 (segment (start 150.59 72) (end 157.5 72) (width 0.2) (layer "F.Cu") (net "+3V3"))
 (segment (start 157 91) (end 154.5 88.5) (width 0.2) (layer "B.Cu") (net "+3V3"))
 (segment (start 154.425 88.5) (end 154.425 78.575) (width 0.2) (layer "B.Cu") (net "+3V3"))
 (segment (start 154.5 88.5) (end 154.425 88.5) (width 0.2) (layer "B.Cu") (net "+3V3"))
 (segment (start 163.58 109.92) (end 169.5 104) (width 0.2) (layer "B.Cu") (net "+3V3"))
 (segment (start 169.5 104) (end 169.5 98.925) (width 0.2) (layer "B.Cu") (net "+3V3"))
 (segment (start 154.425 78.575) (end 157.5 75.5) (width 0.2) (layer "B.Cu") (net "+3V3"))
 (segment (start 161.575 91) (end 157 91) (width 0.2) (layer "B.Cu") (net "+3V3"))
 (segment (start 169.5 98.925) (end 161.575 91) (width 0.2) (layer "B.Cu") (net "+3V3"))
 (segment (start 157.74 109.92) (end 163.58 109.92) (width 0.2) (layer "B.Cu") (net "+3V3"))
 (segment (start 147.6 104) (end 142.5 109.1) (width 0.2) (layer "F.Cu") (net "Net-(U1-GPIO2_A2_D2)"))
 (segment (start 142.5 109.1) (end 142.5 109.92) (width 0.2) (layer "F.Cu") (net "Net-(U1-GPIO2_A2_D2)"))
 (segment (start 138.9 112.235) (end 138.9 104) (width 0.2) (layer "B.Cu") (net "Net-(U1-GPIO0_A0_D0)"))
 (segment (start 141.665 115) (end 138.9 112.235) (width 0.2) (layer "B.Cu") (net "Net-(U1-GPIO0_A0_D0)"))
 (segment (start 148.7 100.544365) (end 148.7 101.455635) (width 0.2) (layer "B.Cu") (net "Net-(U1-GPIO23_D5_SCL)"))
 (segment (start 147.855635 102.3) (end 142.5 102.3) (width 0.2) (layer "B.Cu") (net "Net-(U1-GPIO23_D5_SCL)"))
 (segment (start 148.7 101.455635) (end 147.855635 102.3) (width 0.2) (layer "B.Cu") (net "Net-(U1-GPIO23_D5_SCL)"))
 (segment (start 147 74.41) (end 147 98.844365) (width 0.2) (layer "B.Cu") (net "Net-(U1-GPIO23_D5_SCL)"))
 (segment (start 147 98.844365) (end 148.7 100.544365) (width 0.2) (layer "B.Cu") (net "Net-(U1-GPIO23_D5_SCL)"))
 (segment (start 147 74.41) (end 151.27 70.14) (width 0.2) (layer "B.Cu") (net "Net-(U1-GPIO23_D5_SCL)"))
 (segment (start 136 65) (end 148.67 65) (width 0.2) (layer "F.Cu") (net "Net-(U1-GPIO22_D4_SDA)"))
 (segment (start 131 103.5) (end 131 70) (width 0.2) (layer "F.Cu") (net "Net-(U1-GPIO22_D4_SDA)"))
 (segment (start 131 70) (end 136 65) (width 0.2) (layer "F.Cu") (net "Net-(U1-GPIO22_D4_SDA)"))
 (segment (start 141.84 105.5) (end 133 105.5) (width 0.2) (layer "F.Cu") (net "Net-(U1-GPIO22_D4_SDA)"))
 (segment (start 148.67 65) (end 153.81 70.14) (width 0.2) (layer "F.Cu") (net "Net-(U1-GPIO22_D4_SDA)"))
 (segment (start 142.5 104.84) (end 141.84 105.5) (width 0.2) (layer "F.Cu") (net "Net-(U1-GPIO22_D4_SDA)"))
 (segment (start 133 105.5) (end 131 103.5) (width 0.2) (layer "F.Cu") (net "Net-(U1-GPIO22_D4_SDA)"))
 (segment (start 159.1 106) (end 148.96 106) (width 0.2) (layer "F.Cu") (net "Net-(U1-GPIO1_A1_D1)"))
 (segment (start 161.1 104) (end 159.1 106) (width 0.2) (layer "F.Cu") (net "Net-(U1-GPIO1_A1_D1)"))
 (segment (start 148.96 106) (end 142.5 112.46) (width 0.2) (layer "F.Cu") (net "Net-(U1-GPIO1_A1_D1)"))
 (segment (start 157.5 80.5) (end 141.04 80.5) (width 0.2) (layer "F.Cu") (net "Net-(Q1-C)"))
 (segment (start 141.04 80.5) (end 141 80.54) (width 0.2) (layer "F.Cu") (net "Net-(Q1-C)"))
 (segment (start 159.075 82.075) (end 157.5 80.5) (width 0.2) (layer "B.Cu") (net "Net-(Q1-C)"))
 (segment (start 159.075 88.5) (end 159.075 82.075) (width 0.2) (layer "B.Cu") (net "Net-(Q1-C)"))
 (segment (start 137.75 81.25) (end 137.75 83) (width 0.2) (layer "B.Cu") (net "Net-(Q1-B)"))
 (segment (start 141 78) (end 137.75 81.25) (width 0.2) (layer "B.Cu") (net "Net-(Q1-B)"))
 (segment (start 148.25 84.3) (end 155.2 91.25) (width 0.2) (layer "B.Cu") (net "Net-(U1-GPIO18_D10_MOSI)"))
 (segment (start 148.25 83) (end 148.25 84.3) (width 0.2) (layer "B.Cu") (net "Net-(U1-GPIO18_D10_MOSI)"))
 (segment (start 155.2 104.84) (end 157.74 107.38) (width 0.2) (layer "B.Cu") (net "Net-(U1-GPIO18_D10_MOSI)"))
 (segment (start 155.2 91.25) (end 155.2 104.84) (width 0.2) (layer "B.Cu") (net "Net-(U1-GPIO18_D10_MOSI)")))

